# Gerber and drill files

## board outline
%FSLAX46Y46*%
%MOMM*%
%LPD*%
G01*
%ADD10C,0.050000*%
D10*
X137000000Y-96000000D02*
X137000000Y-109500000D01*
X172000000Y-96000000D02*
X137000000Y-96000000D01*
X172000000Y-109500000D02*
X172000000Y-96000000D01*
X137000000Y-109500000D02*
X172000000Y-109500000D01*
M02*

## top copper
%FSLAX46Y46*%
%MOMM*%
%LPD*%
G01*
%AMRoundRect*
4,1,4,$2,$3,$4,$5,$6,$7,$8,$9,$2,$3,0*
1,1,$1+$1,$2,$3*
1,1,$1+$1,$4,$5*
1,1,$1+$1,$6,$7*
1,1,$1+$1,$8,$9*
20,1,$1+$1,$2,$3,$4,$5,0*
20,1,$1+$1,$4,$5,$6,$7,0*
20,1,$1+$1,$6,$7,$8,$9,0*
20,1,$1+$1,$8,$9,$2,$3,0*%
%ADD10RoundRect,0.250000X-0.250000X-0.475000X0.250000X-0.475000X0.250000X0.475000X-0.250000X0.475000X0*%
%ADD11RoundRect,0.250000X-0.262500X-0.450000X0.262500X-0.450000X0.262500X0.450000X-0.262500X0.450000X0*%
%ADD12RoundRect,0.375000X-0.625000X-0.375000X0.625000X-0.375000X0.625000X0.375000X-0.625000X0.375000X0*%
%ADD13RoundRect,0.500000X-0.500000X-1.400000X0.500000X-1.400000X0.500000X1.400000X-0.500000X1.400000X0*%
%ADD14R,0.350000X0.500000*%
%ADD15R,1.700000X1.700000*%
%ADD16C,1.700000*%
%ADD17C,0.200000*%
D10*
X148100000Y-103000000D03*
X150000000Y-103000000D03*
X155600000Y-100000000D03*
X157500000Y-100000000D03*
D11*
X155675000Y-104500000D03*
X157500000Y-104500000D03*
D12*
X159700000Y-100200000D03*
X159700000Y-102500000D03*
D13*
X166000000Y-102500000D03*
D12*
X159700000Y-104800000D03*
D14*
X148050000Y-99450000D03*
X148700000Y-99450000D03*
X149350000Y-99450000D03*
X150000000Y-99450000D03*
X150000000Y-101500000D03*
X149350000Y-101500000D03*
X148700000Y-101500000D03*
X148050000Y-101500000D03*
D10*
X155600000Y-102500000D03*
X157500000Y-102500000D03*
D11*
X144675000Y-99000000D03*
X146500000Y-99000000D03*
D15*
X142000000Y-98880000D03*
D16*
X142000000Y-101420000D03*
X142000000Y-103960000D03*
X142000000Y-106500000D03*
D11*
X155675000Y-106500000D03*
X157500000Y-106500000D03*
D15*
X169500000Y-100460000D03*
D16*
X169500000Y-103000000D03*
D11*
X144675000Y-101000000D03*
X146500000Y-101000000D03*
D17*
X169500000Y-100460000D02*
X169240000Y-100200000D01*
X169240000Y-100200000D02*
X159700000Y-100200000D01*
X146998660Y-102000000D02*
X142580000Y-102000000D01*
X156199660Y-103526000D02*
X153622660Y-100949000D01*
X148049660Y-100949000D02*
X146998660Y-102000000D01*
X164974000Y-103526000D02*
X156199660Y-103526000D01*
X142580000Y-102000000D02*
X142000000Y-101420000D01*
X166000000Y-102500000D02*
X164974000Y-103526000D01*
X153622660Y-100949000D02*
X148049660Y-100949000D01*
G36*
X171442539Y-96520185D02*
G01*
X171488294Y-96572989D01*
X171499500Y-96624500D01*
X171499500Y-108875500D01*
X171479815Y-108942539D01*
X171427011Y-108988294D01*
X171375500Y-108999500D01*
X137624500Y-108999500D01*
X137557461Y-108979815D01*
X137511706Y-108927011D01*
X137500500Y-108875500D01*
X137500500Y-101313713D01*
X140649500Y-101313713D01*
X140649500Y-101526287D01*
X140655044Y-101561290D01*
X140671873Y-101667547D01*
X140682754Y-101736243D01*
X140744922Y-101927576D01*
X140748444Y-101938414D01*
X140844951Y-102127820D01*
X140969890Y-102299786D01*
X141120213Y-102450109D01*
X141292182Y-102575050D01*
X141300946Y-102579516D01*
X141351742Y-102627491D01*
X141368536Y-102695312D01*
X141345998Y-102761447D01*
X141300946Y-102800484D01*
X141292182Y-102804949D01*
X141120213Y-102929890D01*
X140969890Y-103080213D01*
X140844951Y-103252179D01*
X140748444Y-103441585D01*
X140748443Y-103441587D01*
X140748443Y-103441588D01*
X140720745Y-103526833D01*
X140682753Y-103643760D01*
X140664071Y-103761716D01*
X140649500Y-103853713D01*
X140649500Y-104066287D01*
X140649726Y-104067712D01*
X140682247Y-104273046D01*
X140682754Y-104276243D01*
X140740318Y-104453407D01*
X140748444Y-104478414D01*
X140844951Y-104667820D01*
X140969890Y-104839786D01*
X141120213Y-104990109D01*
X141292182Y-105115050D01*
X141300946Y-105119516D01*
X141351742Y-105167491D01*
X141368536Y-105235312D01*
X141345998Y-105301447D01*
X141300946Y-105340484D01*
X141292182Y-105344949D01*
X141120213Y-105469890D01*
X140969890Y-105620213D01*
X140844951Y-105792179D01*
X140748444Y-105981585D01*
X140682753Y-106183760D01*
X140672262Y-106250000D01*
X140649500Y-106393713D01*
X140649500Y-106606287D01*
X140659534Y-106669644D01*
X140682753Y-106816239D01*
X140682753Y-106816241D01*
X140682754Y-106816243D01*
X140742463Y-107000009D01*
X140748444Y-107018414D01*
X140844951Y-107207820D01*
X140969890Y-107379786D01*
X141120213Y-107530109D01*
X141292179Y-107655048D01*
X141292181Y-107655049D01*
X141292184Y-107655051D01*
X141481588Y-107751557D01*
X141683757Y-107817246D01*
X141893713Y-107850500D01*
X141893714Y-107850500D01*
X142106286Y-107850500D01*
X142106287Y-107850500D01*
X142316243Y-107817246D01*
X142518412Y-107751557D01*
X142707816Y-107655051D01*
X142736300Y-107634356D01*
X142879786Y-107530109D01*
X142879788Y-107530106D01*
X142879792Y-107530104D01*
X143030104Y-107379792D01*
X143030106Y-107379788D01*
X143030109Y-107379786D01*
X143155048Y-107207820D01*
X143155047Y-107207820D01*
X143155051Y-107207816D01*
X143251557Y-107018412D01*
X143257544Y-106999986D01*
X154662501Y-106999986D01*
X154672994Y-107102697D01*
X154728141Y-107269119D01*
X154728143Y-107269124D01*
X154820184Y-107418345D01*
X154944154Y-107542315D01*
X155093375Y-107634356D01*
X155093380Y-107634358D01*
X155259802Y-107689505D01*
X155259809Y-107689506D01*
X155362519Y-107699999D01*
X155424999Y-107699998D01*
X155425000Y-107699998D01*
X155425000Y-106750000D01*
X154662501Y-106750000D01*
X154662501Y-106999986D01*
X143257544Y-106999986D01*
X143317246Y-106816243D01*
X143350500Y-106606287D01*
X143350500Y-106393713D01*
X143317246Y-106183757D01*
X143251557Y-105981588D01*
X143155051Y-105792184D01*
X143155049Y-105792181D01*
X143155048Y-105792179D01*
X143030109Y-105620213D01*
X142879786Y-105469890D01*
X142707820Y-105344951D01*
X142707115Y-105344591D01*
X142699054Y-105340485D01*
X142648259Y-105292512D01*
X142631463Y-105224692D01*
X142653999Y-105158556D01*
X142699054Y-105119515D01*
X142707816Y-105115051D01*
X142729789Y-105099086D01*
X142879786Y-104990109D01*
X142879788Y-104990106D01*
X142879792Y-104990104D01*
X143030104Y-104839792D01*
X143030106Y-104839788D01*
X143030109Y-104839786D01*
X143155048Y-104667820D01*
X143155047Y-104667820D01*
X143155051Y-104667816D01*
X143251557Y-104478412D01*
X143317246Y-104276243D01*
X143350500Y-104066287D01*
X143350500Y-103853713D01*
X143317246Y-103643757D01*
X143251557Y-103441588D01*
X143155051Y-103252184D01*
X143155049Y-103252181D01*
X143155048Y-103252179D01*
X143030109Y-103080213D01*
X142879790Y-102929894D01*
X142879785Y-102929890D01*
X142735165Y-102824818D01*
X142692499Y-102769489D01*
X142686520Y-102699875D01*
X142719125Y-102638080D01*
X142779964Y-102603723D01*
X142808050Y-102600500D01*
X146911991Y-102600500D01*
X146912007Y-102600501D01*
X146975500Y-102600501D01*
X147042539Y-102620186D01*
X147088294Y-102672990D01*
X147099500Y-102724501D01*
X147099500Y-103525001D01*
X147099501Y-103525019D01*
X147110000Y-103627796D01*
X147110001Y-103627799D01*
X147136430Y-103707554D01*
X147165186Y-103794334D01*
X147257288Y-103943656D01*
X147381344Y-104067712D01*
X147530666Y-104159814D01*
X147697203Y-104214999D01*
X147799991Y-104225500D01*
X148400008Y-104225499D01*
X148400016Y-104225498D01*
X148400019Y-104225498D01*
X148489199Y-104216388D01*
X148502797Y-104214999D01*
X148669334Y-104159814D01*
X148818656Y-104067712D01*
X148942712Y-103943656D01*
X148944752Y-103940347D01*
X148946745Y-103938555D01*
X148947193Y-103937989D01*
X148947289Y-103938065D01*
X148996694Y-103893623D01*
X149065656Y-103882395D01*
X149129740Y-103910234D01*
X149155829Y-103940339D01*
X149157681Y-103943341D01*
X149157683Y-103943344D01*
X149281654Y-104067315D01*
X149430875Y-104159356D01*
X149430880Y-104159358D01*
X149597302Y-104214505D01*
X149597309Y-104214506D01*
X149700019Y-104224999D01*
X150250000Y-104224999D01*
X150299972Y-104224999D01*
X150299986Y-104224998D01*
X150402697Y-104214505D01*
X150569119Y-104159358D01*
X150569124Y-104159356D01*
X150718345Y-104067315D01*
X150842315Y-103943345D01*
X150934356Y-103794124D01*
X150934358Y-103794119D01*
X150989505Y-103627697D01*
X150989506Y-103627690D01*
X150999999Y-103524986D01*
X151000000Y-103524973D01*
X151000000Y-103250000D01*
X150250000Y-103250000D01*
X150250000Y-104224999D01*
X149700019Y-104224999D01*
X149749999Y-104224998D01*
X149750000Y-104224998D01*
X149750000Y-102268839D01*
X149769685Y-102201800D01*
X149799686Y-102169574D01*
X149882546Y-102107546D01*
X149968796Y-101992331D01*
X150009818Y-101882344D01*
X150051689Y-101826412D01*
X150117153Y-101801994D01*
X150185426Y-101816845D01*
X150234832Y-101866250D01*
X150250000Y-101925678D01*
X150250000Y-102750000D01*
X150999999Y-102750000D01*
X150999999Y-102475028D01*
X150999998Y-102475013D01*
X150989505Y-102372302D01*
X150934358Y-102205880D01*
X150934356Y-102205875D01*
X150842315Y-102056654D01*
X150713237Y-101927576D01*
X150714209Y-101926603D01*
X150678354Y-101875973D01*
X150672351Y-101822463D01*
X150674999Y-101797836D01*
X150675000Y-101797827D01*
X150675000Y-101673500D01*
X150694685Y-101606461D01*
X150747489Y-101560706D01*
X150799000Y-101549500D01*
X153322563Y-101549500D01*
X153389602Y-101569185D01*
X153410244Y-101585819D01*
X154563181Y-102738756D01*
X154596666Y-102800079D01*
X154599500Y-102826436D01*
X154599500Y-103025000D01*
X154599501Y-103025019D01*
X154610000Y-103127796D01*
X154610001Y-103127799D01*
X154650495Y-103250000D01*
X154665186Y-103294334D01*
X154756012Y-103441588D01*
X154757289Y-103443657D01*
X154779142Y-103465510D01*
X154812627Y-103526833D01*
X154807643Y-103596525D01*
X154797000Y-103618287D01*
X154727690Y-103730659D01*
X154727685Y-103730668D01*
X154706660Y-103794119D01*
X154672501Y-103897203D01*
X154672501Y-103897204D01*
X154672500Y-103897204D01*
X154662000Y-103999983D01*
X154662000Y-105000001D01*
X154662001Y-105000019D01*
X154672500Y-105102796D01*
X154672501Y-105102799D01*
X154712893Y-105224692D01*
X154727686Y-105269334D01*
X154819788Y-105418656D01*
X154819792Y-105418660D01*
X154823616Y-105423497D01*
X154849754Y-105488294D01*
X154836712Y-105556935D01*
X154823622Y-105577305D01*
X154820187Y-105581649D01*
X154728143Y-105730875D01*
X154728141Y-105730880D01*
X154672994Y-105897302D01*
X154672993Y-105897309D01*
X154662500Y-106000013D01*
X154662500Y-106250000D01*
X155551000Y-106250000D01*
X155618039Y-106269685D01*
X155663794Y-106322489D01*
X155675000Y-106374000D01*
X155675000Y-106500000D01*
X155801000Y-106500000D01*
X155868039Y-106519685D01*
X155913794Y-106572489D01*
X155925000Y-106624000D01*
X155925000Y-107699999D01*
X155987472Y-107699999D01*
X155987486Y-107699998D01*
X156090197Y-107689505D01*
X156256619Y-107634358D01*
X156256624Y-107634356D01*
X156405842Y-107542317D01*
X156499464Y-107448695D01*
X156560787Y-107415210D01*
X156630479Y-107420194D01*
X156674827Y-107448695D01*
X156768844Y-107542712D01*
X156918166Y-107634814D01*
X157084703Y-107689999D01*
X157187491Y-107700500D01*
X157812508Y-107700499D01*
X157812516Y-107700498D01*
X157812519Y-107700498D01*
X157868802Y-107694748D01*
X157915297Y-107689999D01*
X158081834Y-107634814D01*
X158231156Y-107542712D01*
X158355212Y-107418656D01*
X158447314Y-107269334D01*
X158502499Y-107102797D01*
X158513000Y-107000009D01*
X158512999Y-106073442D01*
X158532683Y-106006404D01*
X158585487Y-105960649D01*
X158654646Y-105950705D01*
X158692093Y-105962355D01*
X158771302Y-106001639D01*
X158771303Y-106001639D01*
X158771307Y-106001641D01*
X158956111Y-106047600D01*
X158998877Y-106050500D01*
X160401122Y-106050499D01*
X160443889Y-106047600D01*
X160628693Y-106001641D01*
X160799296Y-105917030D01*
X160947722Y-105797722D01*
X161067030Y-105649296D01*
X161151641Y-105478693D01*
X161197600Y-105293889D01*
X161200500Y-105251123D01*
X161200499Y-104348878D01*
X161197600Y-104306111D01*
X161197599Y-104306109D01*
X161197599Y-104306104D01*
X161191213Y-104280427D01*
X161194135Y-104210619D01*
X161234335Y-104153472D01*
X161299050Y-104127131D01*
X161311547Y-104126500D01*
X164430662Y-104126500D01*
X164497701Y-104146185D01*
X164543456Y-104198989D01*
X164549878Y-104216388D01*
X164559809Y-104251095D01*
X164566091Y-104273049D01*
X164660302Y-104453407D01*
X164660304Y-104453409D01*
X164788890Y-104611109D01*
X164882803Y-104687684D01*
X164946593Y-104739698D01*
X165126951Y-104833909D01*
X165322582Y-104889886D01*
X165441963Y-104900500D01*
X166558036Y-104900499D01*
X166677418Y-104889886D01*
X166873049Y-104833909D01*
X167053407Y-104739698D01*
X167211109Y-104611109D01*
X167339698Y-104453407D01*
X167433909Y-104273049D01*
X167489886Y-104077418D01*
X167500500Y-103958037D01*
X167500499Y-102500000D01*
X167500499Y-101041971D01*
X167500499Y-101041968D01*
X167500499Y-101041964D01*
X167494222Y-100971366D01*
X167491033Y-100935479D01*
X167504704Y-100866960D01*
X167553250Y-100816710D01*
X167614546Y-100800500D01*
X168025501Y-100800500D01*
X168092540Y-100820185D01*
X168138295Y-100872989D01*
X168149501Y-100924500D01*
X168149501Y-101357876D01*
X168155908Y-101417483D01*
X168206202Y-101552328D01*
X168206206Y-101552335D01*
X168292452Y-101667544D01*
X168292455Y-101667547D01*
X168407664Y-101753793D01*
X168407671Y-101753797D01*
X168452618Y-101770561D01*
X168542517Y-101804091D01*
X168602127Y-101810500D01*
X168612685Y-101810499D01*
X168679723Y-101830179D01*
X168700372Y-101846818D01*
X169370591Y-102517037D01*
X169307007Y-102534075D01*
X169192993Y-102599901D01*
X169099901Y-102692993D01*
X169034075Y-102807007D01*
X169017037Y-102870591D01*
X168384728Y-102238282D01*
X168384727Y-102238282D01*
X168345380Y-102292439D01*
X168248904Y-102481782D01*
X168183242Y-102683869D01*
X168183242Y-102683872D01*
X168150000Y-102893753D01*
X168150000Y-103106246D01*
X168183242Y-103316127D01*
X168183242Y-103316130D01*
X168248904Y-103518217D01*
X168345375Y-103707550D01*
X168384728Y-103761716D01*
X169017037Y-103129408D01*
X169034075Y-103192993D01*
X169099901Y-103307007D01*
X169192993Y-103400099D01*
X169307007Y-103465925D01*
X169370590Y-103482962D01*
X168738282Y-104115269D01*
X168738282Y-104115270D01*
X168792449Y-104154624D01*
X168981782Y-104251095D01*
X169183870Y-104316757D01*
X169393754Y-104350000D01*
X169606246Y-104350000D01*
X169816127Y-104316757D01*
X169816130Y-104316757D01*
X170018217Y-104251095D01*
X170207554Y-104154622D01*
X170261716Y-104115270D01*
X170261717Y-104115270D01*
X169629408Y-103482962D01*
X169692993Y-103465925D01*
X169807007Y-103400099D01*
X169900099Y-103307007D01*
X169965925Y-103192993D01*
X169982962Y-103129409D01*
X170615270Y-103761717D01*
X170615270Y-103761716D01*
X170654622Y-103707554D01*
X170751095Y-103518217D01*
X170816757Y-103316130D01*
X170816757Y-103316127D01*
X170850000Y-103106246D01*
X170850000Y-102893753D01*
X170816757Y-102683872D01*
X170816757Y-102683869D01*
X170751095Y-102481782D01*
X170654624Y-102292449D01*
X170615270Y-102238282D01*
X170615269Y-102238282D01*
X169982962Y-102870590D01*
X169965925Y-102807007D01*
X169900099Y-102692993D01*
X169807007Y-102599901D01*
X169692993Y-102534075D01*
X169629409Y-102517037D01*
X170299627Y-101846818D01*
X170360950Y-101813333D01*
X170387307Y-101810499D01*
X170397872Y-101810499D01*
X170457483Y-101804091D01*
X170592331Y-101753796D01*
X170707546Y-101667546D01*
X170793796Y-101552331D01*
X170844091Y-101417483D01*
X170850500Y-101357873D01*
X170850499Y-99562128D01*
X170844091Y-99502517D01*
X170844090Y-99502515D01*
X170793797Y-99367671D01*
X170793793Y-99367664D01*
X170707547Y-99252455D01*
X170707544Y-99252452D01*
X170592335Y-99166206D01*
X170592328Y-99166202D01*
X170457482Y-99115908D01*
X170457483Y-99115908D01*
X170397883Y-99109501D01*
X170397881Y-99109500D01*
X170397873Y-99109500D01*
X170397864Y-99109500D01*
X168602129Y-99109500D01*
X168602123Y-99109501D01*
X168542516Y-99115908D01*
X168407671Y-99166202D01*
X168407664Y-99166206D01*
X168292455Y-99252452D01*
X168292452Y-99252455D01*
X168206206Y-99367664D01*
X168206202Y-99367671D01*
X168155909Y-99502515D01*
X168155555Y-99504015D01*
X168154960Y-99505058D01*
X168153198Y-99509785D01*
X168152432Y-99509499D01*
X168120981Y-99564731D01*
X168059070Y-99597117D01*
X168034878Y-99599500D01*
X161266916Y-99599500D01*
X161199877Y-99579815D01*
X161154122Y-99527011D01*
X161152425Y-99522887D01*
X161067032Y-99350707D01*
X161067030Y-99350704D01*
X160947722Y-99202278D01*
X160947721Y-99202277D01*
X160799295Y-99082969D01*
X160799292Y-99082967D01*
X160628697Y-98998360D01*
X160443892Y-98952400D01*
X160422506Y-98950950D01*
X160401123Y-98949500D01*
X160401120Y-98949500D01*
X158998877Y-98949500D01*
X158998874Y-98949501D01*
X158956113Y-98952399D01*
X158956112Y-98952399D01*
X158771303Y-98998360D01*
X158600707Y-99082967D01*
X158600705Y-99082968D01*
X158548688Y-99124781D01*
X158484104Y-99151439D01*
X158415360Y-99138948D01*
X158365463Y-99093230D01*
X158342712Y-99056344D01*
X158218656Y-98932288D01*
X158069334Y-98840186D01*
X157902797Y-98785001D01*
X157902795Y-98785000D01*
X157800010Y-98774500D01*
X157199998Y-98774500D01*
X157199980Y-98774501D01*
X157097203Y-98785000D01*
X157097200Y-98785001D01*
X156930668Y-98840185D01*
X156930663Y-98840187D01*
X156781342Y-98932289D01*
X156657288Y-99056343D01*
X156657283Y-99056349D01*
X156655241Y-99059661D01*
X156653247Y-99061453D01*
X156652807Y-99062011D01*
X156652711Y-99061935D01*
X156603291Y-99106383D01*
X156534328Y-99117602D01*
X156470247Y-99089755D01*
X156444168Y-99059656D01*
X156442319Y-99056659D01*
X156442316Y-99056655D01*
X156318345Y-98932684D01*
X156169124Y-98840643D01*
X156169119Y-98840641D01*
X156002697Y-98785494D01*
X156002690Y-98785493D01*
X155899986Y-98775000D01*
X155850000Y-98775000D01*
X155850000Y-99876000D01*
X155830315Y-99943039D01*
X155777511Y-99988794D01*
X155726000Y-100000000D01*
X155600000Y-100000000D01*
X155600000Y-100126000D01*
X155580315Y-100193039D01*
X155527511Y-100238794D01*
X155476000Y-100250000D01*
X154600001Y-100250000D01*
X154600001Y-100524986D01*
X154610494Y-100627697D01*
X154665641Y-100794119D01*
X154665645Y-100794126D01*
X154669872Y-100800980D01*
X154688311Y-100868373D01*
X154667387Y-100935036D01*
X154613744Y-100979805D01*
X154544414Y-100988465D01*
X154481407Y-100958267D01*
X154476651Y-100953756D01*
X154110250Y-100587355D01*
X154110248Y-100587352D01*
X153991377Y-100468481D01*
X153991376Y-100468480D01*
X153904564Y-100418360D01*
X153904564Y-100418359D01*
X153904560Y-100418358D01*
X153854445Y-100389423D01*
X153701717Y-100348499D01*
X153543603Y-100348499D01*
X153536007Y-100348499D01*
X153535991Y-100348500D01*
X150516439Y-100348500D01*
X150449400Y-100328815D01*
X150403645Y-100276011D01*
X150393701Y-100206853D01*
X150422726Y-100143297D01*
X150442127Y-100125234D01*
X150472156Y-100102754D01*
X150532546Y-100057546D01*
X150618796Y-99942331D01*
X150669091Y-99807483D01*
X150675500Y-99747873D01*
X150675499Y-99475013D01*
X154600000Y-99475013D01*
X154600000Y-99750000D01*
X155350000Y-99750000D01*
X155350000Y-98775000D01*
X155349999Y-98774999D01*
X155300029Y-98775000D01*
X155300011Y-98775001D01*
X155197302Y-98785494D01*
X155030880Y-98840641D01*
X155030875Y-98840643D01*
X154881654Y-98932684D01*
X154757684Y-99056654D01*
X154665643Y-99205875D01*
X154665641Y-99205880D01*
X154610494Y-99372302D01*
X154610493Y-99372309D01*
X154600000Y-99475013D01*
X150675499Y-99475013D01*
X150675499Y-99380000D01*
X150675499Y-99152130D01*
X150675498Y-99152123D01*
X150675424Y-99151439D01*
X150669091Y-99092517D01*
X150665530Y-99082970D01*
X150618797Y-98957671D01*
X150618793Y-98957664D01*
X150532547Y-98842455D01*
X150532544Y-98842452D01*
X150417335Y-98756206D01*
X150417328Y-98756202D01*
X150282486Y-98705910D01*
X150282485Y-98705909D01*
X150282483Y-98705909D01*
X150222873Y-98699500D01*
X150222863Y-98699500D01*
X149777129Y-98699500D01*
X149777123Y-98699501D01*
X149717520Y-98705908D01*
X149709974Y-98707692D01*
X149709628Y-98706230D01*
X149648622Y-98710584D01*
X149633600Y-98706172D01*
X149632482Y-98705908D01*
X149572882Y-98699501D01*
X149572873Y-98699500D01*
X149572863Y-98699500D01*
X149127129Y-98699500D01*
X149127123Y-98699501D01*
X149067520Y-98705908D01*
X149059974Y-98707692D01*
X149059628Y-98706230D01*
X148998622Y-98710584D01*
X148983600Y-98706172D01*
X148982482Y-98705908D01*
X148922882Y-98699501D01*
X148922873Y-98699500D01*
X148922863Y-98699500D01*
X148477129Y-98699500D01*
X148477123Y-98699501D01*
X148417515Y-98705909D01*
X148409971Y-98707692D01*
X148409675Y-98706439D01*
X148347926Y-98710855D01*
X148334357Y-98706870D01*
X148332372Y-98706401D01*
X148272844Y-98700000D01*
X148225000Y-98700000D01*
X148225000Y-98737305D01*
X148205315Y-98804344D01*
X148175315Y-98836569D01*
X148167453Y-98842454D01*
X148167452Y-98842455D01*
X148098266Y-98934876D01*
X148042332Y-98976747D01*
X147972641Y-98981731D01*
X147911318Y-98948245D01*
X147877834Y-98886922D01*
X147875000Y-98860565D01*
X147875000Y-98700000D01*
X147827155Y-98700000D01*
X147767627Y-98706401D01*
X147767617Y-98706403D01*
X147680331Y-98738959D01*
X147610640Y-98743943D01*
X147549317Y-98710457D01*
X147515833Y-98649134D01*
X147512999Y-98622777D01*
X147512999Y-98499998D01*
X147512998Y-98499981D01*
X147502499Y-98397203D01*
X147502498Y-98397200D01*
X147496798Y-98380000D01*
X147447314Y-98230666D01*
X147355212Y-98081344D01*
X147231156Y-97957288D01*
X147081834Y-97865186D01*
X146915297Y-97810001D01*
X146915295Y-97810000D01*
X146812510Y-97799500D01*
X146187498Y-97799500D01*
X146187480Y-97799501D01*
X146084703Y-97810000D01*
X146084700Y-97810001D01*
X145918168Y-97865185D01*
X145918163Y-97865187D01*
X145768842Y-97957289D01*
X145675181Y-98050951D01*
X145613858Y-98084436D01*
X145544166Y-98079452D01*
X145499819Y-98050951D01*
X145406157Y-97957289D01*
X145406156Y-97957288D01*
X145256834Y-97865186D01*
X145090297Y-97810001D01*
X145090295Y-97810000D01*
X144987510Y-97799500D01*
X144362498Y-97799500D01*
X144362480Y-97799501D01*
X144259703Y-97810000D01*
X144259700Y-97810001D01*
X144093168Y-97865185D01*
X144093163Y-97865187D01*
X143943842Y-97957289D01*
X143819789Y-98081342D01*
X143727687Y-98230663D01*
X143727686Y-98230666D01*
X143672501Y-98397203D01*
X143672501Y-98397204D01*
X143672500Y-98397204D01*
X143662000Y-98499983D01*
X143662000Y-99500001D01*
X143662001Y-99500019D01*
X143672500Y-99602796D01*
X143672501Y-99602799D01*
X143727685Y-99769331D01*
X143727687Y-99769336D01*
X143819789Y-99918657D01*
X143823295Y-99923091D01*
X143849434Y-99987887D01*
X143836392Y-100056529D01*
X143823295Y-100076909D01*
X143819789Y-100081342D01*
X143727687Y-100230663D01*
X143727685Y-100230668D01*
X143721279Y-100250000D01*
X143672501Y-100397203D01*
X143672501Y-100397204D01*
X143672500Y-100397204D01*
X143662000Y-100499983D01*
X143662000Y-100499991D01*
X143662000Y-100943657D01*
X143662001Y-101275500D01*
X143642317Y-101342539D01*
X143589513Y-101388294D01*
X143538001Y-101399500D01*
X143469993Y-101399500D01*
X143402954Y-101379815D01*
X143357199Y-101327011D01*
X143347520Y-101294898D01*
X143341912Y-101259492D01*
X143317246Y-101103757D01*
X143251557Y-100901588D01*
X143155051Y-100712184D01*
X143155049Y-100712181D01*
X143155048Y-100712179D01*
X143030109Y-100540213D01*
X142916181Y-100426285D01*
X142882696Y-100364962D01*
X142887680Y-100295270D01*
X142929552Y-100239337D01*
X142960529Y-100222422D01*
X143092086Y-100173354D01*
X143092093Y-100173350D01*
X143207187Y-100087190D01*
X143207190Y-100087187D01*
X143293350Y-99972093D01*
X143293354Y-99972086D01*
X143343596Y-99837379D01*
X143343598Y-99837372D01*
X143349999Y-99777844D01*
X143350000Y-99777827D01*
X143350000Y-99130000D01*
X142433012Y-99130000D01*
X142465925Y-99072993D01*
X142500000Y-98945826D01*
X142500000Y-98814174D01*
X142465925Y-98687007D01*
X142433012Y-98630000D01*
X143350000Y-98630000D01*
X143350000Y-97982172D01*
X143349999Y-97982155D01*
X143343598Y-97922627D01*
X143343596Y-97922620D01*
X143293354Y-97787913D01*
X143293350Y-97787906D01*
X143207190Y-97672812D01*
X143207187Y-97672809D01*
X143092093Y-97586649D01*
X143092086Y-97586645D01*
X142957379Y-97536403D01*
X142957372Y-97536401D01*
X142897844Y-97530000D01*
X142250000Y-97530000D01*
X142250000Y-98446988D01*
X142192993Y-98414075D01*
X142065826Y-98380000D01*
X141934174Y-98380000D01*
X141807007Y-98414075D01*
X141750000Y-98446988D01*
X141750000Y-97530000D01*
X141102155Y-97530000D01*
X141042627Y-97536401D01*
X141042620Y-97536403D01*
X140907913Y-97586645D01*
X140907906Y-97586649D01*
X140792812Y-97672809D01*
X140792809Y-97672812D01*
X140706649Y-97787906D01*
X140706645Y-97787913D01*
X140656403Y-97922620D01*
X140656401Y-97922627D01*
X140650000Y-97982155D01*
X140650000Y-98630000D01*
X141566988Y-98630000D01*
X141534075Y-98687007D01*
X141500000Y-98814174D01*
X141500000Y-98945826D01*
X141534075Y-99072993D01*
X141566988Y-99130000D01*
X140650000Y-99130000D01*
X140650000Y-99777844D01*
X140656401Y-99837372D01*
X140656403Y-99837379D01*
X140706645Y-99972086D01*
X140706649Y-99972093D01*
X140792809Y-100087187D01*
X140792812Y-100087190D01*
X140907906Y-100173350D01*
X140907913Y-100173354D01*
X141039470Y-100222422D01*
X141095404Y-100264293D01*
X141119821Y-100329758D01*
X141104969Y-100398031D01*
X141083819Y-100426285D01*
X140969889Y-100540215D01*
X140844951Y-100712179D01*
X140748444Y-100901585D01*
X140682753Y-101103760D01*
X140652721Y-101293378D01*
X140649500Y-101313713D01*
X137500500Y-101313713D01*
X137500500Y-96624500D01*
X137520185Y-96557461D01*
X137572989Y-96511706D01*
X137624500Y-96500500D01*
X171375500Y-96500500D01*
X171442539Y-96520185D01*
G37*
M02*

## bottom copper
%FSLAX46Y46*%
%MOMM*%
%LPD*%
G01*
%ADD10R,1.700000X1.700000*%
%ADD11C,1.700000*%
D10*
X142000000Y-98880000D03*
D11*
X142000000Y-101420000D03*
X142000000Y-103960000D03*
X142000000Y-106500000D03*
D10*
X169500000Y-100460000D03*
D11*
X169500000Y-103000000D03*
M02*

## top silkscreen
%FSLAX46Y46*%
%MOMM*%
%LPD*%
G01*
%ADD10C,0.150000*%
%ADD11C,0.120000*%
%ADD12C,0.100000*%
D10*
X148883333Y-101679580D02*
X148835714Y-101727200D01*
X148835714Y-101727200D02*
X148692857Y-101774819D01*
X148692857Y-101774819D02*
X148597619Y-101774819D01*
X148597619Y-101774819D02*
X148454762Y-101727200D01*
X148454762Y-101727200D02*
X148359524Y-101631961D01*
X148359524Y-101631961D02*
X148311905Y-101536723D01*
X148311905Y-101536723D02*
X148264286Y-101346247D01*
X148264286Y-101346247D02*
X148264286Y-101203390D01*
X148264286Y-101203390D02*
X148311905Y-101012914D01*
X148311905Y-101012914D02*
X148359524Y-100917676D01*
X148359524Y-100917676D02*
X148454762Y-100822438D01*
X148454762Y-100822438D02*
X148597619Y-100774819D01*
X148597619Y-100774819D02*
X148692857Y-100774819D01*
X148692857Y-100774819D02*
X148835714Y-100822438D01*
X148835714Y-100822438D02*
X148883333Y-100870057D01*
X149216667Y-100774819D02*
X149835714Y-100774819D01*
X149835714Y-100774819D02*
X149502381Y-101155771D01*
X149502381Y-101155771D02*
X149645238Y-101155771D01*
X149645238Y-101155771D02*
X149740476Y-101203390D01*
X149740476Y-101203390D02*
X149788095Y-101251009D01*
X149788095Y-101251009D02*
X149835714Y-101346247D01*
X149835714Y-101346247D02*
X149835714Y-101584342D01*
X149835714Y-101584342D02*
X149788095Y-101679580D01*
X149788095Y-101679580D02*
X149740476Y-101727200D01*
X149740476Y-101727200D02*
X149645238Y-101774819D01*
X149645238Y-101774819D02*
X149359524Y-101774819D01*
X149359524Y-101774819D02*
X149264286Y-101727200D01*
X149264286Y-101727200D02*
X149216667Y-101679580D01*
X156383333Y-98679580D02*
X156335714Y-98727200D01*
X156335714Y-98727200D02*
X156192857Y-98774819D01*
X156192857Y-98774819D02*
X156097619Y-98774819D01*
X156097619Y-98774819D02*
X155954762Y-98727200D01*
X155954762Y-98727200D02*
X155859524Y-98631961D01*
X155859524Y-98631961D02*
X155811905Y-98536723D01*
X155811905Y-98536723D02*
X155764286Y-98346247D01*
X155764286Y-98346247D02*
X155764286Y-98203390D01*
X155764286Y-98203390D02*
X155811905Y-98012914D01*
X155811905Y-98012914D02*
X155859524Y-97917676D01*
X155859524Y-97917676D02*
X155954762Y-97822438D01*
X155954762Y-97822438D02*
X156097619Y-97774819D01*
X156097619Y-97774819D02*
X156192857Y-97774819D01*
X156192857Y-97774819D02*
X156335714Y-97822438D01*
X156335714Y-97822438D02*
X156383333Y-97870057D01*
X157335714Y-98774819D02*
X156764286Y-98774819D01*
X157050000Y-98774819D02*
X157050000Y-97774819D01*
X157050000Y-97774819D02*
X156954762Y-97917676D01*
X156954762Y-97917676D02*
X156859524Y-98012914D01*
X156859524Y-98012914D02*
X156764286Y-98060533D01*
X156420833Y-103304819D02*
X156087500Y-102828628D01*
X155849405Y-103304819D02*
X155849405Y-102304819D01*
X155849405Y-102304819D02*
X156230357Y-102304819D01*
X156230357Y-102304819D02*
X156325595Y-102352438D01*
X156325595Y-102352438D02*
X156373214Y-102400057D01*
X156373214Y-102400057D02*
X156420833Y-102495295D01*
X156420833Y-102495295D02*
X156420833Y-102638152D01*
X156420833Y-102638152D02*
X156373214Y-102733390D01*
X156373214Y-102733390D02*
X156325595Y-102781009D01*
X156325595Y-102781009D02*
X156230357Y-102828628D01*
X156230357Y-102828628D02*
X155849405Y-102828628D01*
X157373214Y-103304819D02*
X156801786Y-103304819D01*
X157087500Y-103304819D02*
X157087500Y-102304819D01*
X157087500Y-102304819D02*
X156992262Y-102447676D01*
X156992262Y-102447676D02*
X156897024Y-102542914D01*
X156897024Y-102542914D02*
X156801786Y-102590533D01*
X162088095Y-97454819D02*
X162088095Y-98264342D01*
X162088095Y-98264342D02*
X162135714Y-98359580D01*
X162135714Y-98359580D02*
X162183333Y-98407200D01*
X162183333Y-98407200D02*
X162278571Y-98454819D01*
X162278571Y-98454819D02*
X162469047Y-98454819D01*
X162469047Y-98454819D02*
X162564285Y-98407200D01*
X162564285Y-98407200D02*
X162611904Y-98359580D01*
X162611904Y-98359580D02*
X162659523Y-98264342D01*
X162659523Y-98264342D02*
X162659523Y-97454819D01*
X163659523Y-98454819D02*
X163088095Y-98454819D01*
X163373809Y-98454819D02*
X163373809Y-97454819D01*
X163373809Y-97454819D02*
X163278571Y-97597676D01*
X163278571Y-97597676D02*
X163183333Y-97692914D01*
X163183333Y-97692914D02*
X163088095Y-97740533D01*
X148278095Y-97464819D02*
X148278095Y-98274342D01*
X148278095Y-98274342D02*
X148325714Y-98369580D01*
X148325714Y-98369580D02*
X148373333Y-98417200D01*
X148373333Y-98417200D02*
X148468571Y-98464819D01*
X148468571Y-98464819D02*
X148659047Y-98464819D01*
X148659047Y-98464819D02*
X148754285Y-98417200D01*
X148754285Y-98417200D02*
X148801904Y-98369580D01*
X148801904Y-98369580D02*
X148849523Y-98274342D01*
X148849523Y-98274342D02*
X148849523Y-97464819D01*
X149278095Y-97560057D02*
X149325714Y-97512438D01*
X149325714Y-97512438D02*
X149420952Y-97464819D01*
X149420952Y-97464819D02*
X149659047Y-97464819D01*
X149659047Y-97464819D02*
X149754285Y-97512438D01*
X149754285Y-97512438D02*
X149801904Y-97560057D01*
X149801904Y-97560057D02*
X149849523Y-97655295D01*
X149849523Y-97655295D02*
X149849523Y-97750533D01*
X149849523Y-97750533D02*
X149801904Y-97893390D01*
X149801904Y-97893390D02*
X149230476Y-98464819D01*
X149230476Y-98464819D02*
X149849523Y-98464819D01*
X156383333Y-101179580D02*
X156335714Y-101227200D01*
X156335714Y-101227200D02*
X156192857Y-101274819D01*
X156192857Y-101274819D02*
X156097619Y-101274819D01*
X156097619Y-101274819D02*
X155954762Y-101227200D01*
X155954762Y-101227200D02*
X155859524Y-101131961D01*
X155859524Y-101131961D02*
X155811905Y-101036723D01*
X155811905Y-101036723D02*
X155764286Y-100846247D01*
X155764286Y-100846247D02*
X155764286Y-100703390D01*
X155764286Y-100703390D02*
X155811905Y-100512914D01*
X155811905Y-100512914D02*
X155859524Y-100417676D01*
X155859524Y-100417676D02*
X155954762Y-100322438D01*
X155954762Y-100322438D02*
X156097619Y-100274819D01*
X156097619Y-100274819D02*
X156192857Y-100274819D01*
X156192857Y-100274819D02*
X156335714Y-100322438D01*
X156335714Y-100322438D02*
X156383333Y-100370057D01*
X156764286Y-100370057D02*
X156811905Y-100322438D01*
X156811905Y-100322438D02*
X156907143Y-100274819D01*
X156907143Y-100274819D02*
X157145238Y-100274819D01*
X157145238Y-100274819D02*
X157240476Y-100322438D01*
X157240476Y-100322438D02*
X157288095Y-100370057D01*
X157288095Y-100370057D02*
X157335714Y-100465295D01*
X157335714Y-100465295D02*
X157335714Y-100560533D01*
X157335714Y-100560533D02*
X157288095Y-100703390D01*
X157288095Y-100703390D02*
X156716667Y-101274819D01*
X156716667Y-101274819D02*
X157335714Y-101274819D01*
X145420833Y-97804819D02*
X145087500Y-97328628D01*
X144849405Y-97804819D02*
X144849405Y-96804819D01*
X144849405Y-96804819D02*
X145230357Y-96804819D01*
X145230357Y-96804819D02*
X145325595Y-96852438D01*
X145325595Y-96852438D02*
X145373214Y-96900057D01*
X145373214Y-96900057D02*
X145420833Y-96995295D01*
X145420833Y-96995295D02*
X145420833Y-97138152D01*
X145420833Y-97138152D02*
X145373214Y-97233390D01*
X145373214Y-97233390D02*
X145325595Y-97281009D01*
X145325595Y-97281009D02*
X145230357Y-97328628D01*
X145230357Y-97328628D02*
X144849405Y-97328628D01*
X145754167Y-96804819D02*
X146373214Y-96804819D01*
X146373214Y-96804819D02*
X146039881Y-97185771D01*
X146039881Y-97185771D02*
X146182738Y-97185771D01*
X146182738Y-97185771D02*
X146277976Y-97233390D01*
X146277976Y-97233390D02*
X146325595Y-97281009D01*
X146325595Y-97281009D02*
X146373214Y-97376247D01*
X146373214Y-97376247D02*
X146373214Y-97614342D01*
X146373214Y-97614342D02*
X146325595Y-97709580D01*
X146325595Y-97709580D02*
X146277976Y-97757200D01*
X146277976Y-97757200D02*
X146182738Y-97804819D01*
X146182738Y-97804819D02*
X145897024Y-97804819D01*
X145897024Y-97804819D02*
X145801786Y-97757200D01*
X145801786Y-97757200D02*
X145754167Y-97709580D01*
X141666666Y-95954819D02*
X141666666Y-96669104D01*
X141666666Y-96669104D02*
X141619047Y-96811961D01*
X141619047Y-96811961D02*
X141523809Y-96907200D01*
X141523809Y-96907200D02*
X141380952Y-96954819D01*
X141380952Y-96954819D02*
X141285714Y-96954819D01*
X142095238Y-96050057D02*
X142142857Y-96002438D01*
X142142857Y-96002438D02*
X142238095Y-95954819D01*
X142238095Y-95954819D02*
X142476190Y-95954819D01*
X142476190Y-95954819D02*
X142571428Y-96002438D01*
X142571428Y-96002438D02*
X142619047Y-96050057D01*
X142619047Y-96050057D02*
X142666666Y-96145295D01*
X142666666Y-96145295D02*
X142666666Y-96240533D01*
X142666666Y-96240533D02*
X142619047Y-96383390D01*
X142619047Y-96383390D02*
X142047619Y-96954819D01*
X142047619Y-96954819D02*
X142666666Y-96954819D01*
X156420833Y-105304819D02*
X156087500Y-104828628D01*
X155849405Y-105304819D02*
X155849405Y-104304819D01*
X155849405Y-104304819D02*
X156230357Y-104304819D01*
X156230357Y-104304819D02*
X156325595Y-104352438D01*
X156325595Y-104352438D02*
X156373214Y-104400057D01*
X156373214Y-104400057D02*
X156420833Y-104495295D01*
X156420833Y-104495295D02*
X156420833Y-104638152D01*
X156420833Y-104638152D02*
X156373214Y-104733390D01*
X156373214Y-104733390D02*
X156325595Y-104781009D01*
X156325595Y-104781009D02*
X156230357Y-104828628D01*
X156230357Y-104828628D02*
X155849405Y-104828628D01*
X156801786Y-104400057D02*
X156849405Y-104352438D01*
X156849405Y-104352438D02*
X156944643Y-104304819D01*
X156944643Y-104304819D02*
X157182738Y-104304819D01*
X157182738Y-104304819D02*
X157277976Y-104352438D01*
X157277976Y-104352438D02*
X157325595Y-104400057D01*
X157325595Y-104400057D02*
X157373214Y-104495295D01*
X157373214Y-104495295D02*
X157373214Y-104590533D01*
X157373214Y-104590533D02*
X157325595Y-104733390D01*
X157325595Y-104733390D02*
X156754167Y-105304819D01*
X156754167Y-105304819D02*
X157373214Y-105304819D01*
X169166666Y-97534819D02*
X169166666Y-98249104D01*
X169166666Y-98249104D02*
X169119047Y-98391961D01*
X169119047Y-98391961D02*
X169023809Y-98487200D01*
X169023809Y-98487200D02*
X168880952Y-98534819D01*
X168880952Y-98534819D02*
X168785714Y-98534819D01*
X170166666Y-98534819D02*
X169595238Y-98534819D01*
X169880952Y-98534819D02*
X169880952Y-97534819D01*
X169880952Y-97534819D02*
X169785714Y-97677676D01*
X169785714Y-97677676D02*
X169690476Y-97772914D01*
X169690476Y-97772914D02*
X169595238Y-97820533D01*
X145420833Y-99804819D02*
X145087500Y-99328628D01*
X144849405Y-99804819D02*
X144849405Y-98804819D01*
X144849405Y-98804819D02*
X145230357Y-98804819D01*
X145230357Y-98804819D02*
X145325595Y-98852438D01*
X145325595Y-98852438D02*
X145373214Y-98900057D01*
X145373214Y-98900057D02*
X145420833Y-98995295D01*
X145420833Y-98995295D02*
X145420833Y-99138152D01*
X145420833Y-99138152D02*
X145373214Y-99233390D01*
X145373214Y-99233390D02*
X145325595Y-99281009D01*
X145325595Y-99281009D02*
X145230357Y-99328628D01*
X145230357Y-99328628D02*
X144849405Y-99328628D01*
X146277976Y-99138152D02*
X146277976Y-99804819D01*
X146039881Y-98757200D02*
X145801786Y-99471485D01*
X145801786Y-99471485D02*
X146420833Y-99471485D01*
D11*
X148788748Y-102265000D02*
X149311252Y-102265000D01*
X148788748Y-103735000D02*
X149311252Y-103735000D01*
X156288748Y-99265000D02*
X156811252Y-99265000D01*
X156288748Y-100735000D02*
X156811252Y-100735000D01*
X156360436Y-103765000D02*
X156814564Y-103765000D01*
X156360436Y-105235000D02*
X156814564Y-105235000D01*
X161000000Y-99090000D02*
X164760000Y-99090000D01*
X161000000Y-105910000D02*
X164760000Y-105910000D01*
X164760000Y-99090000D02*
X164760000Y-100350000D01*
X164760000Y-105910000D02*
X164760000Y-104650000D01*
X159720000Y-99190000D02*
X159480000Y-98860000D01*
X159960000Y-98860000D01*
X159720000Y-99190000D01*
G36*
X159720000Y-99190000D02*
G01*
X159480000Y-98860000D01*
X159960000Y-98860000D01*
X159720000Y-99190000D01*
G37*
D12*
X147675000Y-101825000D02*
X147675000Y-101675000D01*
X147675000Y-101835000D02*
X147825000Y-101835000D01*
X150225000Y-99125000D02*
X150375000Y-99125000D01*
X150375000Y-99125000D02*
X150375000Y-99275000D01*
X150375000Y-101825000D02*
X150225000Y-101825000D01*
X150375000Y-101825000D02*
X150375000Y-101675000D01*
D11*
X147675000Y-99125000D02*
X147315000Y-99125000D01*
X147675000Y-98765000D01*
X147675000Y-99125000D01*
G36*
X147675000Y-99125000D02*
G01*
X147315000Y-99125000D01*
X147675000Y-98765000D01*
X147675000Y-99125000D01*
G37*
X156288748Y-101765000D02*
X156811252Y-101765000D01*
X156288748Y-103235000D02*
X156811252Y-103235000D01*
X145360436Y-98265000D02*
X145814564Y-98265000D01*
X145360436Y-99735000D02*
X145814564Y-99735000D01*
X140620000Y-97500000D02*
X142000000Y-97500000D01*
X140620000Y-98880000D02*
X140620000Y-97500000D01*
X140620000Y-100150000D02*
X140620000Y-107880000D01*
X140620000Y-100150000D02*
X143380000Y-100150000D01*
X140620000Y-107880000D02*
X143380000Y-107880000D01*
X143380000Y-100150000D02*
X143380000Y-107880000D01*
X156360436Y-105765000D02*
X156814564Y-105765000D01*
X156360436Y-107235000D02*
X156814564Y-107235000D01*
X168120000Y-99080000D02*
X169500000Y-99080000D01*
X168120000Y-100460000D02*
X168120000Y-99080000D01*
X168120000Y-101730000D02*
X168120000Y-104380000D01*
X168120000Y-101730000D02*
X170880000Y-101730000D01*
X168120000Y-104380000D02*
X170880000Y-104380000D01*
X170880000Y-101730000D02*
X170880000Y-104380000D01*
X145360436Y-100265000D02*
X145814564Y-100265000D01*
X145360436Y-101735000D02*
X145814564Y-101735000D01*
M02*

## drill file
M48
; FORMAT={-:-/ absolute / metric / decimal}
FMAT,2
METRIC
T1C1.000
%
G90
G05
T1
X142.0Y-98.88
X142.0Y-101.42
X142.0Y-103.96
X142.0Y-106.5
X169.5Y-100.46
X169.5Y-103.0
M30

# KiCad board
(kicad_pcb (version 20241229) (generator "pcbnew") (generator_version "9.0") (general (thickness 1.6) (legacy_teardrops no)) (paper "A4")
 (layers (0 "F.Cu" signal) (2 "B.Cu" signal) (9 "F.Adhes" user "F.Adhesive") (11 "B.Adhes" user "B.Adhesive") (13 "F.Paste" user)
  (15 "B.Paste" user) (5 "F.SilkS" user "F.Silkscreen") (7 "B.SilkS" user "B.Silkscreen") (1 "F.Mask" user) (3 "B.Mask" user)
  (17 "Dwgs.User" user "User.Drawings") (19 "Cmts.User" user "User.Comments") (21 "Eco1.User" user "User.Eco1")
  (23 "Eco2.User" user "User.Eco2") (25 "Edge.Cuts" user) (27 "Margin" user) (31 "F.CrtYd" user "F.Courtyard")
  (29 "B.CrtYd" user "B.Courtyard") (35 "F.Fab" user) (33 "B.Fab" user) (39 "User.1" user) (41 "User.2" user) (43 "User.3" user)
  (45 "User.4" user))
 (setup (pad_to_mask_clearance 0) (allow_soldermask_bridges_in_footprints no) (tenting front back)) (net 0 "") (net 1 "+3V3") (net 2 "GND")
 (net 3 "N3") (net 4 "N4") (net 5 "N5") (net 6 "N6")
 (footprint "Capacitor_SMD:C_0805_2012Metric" (layer "F.Cu") (at 149.05 103)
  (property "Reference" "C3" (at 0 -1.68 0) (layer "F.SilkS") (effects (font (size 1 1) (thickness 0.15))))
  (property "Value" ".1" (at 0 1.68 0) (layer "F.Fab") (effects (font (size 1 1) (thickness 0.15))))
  (fp_line (start -0.261252 -0.735) (end 0.261252 -0.735) (stroke (width 0.12) (type solid)) (layer "F.SilkS"))
  (fp_line (start -0.261252 0.735) (end 0.261252 0.735) (stroke (width 0.12) (type solid)) (layer "F.SilkS"))
  (pad "1" smd roundrect (at -0.95 0) (size 1 1.45) (layers "F.Cu" "F.Mask" "F.Paste") (roundrect_rratio 0.25) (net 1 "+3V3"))
  (pad "2" smd roundrect (at 0.95 0) (size 1 1.45) (layers "F.Cu" "F.Mask" "F.Paste") (roundrect_rratio 0.25) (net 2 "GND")))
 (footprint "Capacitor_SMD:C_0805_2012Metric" (layer "F.Cu") (at 156.55 100)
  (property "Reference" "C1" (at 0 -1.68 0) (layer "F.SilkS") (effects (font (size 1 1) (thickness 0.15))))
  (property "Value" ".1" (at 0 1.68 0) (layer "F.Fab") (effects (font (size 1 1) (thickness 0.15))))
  (fp_line (start -0.261252 -0.735) (end 0.261252 -0.735) (stroke (width 0.12) (type solid)) (layer "F.SilkS"))
  (fp_line (start -0.261252 0.735) (end 0.261252 0.735) (stroke (width 0.12) (type solid)) (layer "F.SilkS"))
  (pad "1" smd roundrect (at -0.95 0) (size 1 1.45) (layers "F.Cu" "F.Mask" "F.Paste") (roundrect_rratio 0.25) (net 2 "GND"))
  (pad "2" smd roundrect (at 0.95 0) (size 1 1.45) (layers "F.Cu" "F.Mask" "F.Paste") (roundrect_rratio 0.25) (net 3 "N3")))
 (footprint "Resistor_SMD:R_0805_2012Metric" (layer "F.Cu") (at 156.5875 104.5)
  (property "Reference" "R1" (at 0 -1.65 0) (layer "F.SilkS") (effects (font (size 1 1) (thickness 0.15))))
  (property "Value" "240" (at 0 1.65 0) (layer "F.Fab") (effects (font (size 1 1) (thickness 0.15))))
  (fp_line (start -0.227064 -0.735) (end 0.227064 -0.735) (stroke (width 0.12) (type solid)) (layer "F.SilkS"))
  (fp_line (start -0.227064 0.735) (end 0.227064 0.735) (stroke (width 0.12) (type solid)) (layer "F.SilkS"))
  (pad "1" smd roundrect (at -0.9125 0) (size 1.025 1.4) (layers "F.Cu" "F.Mask" "F.Paste") (roundrect_rratio 0.243902) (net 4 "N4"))
  (pad "2" smd roundrect (at 0.9125 0) (size 1.025 1.4) (layers "F.Cu" "F.Mask" "F.Paste") (roundrect_rratio 0.243902) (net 1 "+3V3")))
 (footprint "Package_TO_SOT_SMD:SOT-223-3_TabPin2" (layer "F.Cu") (at 162.85 102.5)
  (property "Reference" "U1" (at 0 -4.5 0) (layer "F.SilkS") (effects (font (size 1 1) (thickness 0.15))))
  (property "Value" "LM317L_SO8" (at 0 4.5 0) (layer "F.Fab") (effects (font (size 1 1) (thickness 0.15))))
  (fp_line (start -1.85 -3.41) (end 1.91 -3.41) (stroke (width 0.12) (type solid)) (layer "F.SilkS"))
  (fp_line (start -1.85 3.41) (end 1.91 3.41) (stroke (width 0.12) (type solid)) (layer "F.SilkS"))
  (fp_line (start 1.91 -3.41) (end 1.91 -2.15) (stroke (width 0.12) (type solid)) (layer "F.SilkS"))
  (fp_line (start 1.91 3.41) (end 1.91 2.15) (stroke (width 0.12) (type solid)) (layer "F.SilkS"))
  (fp_poly
   (pts (xy -3.13 -3.31) (xy -3.37 -3.64) (xy -2.89 -3.64) (xy -3.13 -3.31)) (stroke (width 0.12) (type solid)) (fill yes) (layer "F.SilkS"))
  (pad "1" smd roundrect (at -3.15 -2.3) (size 2 1.5) (layers "F.Cu" "F.Mask" "F.Paste") (roundrect_rratio 0.25) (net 3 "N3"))
  (pad "2" smd roundrect (at -3.15 0) (size 2 1.5) (layers "F.Cu" "F.Mask" "F.Paste") (roundrect_rratio 0.25) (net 1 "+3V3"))
  (pad "2" smd roundrect (at 3.15 0) (size 2 3.8) (layers "F.Cu" "F.Mask" "F.Paste") (roundrect_rratio 0.25) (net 1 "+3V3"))
  (pad "3" smd roundrect (at -3.15 2.3) (size 2 1.5) (layers "F.Cu" "F.Mask" "F.Paste") (roundrect_rratio 0.25) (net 1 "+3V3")))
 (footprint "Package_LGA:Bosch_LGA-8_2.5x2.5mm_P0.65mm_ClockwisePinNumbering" (layer "F.Cu") (at 149.025 100.475)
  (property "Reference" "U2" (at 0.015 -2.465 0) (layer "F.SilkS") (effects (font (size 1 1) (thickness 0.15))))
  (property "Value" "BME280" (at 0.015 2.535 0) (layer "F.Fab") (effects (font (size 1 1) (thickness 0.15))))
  (fp_line (start -1.35 1.35) (end -1.35 1.2) (stroke (width 0.1) (type solid)) (layer "F.SilkS"))
  (fp_line (start -1.35 1.36) (end -1.2 1.36) (stroke (width 0.1) (type solid)) (layer "F.SilkS"))
  (fp_line (start 1.2 -1.35) (end 1.35 -1.35) (stroke (width 0.1) (type solid)) (layer "F.SilkS"))
  (fp_line (start 1.35 -1.35) (end 1.35 -1.2) (stroke (width 0.1) (type solid)) (layer "F.SilkS"))
  (fp_line (start 1.35 1.35) (end 1.2 1.35) (stroke (width 0.1) (type solid)) (layer "F.SilkS"))
  (fp_line (start 1.35 1.35) (end 1.35 1.2) (stroke (width 0.1) (type solid)) (layer "F.SilkS"))
  (fp_poly
   (pts (xy -1.35 -1.35) (xy -1.71 -1.35) (xy -1.35 -1.71) (xy -1.35 -1.35)) (stroke (width 0.12) (type solid)) (fill yes) (layer "F.SilkS"))
  (pad "1" smd rect (at -0.975 -1.025 90) (size 0.5 0.35) (layers "F.Cu" "F.Mask" "F.Paste") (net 2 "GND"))
  (pad "2" smd rect (at -0.325 -1.025 90) (size 0.5 0.35) (layers "F.Cu" "F.Mask" "F.Paste") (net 1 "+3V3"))
  (pad "3" smd rect (at 0.325 -1.025 90) (size 0.5 0.35) (layers "F.Cu" "F.Mask" "F.Paste") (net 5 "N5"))
  (pad "4" smd rect (at 0.975 -1.025 90) (size 0.5 0.35) (layers "F.Cu" "F.Mask" "F.Paste") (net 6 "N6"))
  (pad "5" smd rect (at 0.975 1.025 90) (size 0.5 0.35) (layers "F.Cu" "F.Mask" "F.Paste") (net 2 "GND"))
  (pad "6" smd rect (at 0.325 1.025 90) (size 0.5 0.35) (layers "F.Cu" "F.Mask" "F.Paste") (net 1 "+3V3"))
  (pad "7" smd rect (at -0.325 1.025 90) (size 0.5 0.35) (layers "F.Cu" "F.Mask" "F.Paste") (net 2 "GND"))
  (pad "8" smd rect (at -0.975 1.025 90) (size 0.5 0.35) (layers "F.Cu" "F.Mask" "F.Paste") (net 1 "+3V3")))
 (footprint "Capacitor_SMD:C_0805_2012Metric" (layer "F.Cu") (at 156.55 102.5)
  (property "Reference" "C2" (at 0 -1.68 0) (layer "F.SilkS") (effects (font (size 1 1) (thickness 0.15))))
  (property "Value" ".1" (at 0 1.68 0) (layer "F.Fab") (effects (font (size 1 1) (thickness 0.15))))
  (fp_line (start -0.261252 -0.735) (end 0.261252 -0.735) (stroke (width 0.12) (type solid)) (layer "F.SilkS"))
  (fp_line (start -0.261252 0.735) (end 0.261252 0.735) (stroke (width 0.12) (type solid)) (layer "F.SilkS"))
  (pad "1" smd roundrect (at -0.95 0) (size 1 1.45) (layers "F.Cu" "F.Mask" "F.Paste") (roundrect_rratio 0.25) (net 1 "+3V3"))
  (pad "2" smd roundrect (at 0.95 0) (size 1 1.45) (layers "F.Cu" "F.Mask" "F.Paste") (roundrect_rratio 0.25) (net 2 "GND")))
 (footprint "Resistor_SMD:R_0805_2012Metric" (layer "F.Cu") (at 145.5875 99)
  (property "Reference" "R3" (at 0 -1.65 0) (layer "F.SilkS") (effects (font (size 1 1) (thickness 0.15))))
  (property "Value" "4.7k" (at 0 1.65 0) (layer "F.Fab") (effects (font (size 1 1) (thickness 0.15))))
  (fp_line (start -0.227064 -0.735) (end 0.227064 -0.735) (stroke (width 0.12) (type solid)) (layer "F.SilkS"))
  (fp_line (start -0.227064 0.735) (end 0.227064 0.735) (stroke (width 0.12) (type solid)) (layer "F.SilkS"))
  (pad "1" smd roundrect (at -0.9125 0) (size 1.025 1.4) (layers "F.Cu" "F.Mask" "F.Paste") (roundrect_rratio 0.243902) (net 1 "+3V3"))
  (pad "2" smd roundrect (at 0.9125 0) (size 1.025 1.4) (layers "F.Cu" "F.Mask" "F.Paste") (roundrect_rratio 0.243902) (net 6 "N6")))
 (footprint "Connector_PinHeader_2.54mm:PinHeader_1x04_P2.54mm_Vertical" (layer "F.Cu") (at 142 98.88)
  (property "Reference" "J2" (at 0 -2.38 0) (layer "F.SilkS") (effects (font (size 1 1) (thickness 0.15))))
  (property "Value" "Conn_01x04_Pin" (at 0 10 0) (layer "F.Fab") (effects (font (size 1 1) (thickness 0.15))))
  (fp_line (start -1.38 -1.38) (end 0 -1.38) (stroke (width 0.12) (type solid)) (layer "F.SilkS"))
  (fp_line (start -1.38 0) (end -1.38 -1.38) (stroke (width 0.12) (type solid)) (layer "F.SilkS"))
  (fp_line (start -1.38 1.27) (end -1.38 9) (stroke (width 0.12) (type solid)) (layer "F.SilkS"))
  (fp_line (start -1.38 1.27) (end 1.38 1.27) (stroke (width 0.12) (type solid)) (layer "F.SilkS"))
  (fp_line (start -1.38 9) (end 1.38 9) (stroke (width 0.12) (type solid)) (layer "F.SilkS"))
  (fp_line (start 1.38 1.27) (end 1.38 9) (stroke (width 0.12) (type solid)) (layer "F.SilkS"))
  (pad "1" thru_hole rect (at 0 0) (size 1.7 1.7) (drill 1) (layers "*.Cu" "*.Mask") (remove_unused_layers no) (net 2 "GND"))
  (pad "2" thru_hole circle (at 0 2.54) (size 1.7 1.7) (drill 1) (layers "*.Cu" "*.Mask") (remove_unused_layers no) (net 1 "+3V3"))
  (pad "3" thru_hole circle (at 0 5.08) (size 1.7 1.7) (drill 1) (layers "*.Cu" "*.Mask") (remove_unused_layers no) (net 5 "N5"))
  (pad "4" thru_hole circle (at 0 7.62) (size 1.7 1.7) (drill 1) (layers "*.Cu" "*.Mask") (remove_unused_layers no) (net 6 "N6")))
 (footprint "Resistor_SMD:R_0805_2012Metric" (layer "F.Cu") (at 156.5875 106.5)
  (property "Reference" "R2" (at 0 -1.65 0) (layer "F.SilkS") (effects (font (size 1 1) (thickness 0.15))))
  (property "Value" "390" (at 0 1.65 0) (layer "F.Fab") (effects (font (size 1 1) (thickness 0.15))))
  (fp_line (start -0.227064 -0.735) (end 0.227064 -0.735) (stroke (width 0.12) (type solid)) (layer "F.SilkS"))
  (fp_line (start -0.227064 0.735) (end 0.227064 0.735) (stroke (width 0.12) (type solid)) (layer "F.SilkS"))
  (pad "1" smd roundrect (at -0.9125 0) (size 1.025 1.4) (layers "F.Cu" "F.Mask" "F.Paste") (roundrect_rratio 0.243902) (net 2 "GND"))
  (pad "2" smd roundrect (at 0.9125 0) (size 1.025 1.4) (layers "F.Cu" "F.Mask" "F.Paste") (roundrect_rratio 0.243902) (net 4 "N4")))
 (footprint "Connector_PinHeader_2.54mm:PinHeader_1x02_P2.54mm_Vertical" (layer "F.Cu") (at 169.5 100.46)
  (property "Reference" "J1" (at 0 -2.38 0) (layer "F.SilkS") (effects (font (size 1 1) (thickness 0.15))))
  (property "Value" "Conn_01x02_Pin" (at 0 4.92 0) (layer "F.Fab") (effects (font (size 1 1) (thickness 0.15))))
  (fp_line (start -1.38 -1.38) (end 0 -1.38) (stroke (width 0.12) (type solid)) (layer "F.SilkS"))
  (fp_line (start -1.38 0) (end -1.38 -1.38) (stroke (width 0.12) (type solid)) (layer "F.SilkS"))
  (fp_line (start -1.38 1.27) (end -1.38 3.92) (stroke (width 0.12) (type solid)) (layer "F.SilkS"))
  (fp_line (start -1.38 1.27) (end 1.38 1.27) (stroke (width 0.12) (type solid)) (layer "F.SilkS"))
  (fp_line (start -1.38 3.92) (end 1.38 3.92) (stroke (width 0.12) (type solid)) (layer "F.SilkS"))
  (fp_line (start 1.38 1.27) (end 1.38 3.92) (stroke (width 0.12) (type solid)) (layer "F.SilkS"))
  (pad "1" thru_hole rect (at 0 0) (size 1.7 1.7) (drill 1) (layers "*.Cu" "*.Mask") (remove_unused_layers no) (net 3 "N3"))
  (pad "2" thru_hole circle (at 0 2.54) (size 1.7 1.7) (drill 1) (layers "*.Cu" "*.Mask") (remove_unused_layers no) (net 2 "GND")))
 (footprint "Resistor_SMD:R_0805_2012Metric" (layer "F.Cu") (at 145.5875 101)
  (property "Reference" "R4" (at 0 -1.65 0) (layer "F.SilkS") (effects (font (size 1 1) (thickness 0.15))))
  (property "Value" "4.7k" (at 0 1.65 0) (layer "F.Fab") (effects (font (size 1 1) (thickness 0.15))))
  (fp_line (start -0.227064 -0.735) (end 0.227064 -0.735) (stroke (width 0.12) (type solid)) (layer "F.SilkS"))
  (fp_line (start -0.227064 0.735) (end 0.227064 0.735) (stroke (width 0.12) (type solid)) (layer "F.SilkS"))
  (pad "1" smd roundrect (at -0.9125 0) (size 1.025 1.4) (layers "F.Cu" "F.Mask" "F.Paste") (roundrect_rratio 0.243902) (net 1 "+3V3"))
  (pad "2" smd roundrect (at 0.9125 0) (size 1.025 1.4) (layers "F.Cu" "F.Mask" "F.Paste") (roundrect_rratio 0.243902) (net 5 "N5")))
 (gr_line (start 137 96) (end 137 109.5) (stroke (width 0.05) (type default)) (layer "Edge.Cuts"))
 (gr_line (start 172 96) (end 137 96) (stroke (width 0.05) (type default)) (layer "Edge.Cuts"))
 (gr_line (start 172 109.5) (end 172 96) (stroke (width 0.05) (type default)) (layer "Edge.Cuts"))
 (gr_line (start 137 109.5) (end 172 109.5) (stroke (width 0.05) (type default)) (layer "Edge.Cuts"))
 (segment (start 169.5 100.46) (end 169.24 100.2) (width 0.2) (layer "F.Cu") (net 3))
 (segment (start 169.24 100.2) (end 159.7 100.2) (width 0.2) (layer "F.Cu") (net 3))
 (segment (start 146.99866 102) (end 142.58 102) (width 0.2) (layer "F.Cu") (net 1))
 (segment (start 156.19966 103.526) (end 153.62266 100.949) (width 0.2) (layer "F.Cu") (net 1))
 (segment (start 148.04966 100.949) (end 146.99866 102) (width 0.2) (layer "F.Cu") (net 1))
 (segment (start 164.974 103.526) (end 156.19966 103.526) (width 0.2) (layer "F.Cu") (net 1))
 (segment (start 142.58 102) (end 142 101.42) (width 0.2) (layer "F.Cu") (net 1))
 (segment (start 166 102.5) (end 164.974 103.526) (width 0.2) (layer "F.Cu") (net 1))
 (segment (start 153.62266 100.949) (end 148.04966 100.949) (width 0.2) (layer "F.Cu") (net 1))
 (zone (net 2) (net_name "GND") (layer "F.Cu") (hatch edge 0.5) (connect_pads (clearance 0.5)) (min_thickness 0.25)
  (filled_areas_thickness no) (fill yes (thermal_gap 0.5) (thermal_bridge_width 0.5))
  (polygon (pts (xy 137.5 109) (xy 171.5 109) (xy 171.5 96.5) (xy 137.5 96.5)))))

